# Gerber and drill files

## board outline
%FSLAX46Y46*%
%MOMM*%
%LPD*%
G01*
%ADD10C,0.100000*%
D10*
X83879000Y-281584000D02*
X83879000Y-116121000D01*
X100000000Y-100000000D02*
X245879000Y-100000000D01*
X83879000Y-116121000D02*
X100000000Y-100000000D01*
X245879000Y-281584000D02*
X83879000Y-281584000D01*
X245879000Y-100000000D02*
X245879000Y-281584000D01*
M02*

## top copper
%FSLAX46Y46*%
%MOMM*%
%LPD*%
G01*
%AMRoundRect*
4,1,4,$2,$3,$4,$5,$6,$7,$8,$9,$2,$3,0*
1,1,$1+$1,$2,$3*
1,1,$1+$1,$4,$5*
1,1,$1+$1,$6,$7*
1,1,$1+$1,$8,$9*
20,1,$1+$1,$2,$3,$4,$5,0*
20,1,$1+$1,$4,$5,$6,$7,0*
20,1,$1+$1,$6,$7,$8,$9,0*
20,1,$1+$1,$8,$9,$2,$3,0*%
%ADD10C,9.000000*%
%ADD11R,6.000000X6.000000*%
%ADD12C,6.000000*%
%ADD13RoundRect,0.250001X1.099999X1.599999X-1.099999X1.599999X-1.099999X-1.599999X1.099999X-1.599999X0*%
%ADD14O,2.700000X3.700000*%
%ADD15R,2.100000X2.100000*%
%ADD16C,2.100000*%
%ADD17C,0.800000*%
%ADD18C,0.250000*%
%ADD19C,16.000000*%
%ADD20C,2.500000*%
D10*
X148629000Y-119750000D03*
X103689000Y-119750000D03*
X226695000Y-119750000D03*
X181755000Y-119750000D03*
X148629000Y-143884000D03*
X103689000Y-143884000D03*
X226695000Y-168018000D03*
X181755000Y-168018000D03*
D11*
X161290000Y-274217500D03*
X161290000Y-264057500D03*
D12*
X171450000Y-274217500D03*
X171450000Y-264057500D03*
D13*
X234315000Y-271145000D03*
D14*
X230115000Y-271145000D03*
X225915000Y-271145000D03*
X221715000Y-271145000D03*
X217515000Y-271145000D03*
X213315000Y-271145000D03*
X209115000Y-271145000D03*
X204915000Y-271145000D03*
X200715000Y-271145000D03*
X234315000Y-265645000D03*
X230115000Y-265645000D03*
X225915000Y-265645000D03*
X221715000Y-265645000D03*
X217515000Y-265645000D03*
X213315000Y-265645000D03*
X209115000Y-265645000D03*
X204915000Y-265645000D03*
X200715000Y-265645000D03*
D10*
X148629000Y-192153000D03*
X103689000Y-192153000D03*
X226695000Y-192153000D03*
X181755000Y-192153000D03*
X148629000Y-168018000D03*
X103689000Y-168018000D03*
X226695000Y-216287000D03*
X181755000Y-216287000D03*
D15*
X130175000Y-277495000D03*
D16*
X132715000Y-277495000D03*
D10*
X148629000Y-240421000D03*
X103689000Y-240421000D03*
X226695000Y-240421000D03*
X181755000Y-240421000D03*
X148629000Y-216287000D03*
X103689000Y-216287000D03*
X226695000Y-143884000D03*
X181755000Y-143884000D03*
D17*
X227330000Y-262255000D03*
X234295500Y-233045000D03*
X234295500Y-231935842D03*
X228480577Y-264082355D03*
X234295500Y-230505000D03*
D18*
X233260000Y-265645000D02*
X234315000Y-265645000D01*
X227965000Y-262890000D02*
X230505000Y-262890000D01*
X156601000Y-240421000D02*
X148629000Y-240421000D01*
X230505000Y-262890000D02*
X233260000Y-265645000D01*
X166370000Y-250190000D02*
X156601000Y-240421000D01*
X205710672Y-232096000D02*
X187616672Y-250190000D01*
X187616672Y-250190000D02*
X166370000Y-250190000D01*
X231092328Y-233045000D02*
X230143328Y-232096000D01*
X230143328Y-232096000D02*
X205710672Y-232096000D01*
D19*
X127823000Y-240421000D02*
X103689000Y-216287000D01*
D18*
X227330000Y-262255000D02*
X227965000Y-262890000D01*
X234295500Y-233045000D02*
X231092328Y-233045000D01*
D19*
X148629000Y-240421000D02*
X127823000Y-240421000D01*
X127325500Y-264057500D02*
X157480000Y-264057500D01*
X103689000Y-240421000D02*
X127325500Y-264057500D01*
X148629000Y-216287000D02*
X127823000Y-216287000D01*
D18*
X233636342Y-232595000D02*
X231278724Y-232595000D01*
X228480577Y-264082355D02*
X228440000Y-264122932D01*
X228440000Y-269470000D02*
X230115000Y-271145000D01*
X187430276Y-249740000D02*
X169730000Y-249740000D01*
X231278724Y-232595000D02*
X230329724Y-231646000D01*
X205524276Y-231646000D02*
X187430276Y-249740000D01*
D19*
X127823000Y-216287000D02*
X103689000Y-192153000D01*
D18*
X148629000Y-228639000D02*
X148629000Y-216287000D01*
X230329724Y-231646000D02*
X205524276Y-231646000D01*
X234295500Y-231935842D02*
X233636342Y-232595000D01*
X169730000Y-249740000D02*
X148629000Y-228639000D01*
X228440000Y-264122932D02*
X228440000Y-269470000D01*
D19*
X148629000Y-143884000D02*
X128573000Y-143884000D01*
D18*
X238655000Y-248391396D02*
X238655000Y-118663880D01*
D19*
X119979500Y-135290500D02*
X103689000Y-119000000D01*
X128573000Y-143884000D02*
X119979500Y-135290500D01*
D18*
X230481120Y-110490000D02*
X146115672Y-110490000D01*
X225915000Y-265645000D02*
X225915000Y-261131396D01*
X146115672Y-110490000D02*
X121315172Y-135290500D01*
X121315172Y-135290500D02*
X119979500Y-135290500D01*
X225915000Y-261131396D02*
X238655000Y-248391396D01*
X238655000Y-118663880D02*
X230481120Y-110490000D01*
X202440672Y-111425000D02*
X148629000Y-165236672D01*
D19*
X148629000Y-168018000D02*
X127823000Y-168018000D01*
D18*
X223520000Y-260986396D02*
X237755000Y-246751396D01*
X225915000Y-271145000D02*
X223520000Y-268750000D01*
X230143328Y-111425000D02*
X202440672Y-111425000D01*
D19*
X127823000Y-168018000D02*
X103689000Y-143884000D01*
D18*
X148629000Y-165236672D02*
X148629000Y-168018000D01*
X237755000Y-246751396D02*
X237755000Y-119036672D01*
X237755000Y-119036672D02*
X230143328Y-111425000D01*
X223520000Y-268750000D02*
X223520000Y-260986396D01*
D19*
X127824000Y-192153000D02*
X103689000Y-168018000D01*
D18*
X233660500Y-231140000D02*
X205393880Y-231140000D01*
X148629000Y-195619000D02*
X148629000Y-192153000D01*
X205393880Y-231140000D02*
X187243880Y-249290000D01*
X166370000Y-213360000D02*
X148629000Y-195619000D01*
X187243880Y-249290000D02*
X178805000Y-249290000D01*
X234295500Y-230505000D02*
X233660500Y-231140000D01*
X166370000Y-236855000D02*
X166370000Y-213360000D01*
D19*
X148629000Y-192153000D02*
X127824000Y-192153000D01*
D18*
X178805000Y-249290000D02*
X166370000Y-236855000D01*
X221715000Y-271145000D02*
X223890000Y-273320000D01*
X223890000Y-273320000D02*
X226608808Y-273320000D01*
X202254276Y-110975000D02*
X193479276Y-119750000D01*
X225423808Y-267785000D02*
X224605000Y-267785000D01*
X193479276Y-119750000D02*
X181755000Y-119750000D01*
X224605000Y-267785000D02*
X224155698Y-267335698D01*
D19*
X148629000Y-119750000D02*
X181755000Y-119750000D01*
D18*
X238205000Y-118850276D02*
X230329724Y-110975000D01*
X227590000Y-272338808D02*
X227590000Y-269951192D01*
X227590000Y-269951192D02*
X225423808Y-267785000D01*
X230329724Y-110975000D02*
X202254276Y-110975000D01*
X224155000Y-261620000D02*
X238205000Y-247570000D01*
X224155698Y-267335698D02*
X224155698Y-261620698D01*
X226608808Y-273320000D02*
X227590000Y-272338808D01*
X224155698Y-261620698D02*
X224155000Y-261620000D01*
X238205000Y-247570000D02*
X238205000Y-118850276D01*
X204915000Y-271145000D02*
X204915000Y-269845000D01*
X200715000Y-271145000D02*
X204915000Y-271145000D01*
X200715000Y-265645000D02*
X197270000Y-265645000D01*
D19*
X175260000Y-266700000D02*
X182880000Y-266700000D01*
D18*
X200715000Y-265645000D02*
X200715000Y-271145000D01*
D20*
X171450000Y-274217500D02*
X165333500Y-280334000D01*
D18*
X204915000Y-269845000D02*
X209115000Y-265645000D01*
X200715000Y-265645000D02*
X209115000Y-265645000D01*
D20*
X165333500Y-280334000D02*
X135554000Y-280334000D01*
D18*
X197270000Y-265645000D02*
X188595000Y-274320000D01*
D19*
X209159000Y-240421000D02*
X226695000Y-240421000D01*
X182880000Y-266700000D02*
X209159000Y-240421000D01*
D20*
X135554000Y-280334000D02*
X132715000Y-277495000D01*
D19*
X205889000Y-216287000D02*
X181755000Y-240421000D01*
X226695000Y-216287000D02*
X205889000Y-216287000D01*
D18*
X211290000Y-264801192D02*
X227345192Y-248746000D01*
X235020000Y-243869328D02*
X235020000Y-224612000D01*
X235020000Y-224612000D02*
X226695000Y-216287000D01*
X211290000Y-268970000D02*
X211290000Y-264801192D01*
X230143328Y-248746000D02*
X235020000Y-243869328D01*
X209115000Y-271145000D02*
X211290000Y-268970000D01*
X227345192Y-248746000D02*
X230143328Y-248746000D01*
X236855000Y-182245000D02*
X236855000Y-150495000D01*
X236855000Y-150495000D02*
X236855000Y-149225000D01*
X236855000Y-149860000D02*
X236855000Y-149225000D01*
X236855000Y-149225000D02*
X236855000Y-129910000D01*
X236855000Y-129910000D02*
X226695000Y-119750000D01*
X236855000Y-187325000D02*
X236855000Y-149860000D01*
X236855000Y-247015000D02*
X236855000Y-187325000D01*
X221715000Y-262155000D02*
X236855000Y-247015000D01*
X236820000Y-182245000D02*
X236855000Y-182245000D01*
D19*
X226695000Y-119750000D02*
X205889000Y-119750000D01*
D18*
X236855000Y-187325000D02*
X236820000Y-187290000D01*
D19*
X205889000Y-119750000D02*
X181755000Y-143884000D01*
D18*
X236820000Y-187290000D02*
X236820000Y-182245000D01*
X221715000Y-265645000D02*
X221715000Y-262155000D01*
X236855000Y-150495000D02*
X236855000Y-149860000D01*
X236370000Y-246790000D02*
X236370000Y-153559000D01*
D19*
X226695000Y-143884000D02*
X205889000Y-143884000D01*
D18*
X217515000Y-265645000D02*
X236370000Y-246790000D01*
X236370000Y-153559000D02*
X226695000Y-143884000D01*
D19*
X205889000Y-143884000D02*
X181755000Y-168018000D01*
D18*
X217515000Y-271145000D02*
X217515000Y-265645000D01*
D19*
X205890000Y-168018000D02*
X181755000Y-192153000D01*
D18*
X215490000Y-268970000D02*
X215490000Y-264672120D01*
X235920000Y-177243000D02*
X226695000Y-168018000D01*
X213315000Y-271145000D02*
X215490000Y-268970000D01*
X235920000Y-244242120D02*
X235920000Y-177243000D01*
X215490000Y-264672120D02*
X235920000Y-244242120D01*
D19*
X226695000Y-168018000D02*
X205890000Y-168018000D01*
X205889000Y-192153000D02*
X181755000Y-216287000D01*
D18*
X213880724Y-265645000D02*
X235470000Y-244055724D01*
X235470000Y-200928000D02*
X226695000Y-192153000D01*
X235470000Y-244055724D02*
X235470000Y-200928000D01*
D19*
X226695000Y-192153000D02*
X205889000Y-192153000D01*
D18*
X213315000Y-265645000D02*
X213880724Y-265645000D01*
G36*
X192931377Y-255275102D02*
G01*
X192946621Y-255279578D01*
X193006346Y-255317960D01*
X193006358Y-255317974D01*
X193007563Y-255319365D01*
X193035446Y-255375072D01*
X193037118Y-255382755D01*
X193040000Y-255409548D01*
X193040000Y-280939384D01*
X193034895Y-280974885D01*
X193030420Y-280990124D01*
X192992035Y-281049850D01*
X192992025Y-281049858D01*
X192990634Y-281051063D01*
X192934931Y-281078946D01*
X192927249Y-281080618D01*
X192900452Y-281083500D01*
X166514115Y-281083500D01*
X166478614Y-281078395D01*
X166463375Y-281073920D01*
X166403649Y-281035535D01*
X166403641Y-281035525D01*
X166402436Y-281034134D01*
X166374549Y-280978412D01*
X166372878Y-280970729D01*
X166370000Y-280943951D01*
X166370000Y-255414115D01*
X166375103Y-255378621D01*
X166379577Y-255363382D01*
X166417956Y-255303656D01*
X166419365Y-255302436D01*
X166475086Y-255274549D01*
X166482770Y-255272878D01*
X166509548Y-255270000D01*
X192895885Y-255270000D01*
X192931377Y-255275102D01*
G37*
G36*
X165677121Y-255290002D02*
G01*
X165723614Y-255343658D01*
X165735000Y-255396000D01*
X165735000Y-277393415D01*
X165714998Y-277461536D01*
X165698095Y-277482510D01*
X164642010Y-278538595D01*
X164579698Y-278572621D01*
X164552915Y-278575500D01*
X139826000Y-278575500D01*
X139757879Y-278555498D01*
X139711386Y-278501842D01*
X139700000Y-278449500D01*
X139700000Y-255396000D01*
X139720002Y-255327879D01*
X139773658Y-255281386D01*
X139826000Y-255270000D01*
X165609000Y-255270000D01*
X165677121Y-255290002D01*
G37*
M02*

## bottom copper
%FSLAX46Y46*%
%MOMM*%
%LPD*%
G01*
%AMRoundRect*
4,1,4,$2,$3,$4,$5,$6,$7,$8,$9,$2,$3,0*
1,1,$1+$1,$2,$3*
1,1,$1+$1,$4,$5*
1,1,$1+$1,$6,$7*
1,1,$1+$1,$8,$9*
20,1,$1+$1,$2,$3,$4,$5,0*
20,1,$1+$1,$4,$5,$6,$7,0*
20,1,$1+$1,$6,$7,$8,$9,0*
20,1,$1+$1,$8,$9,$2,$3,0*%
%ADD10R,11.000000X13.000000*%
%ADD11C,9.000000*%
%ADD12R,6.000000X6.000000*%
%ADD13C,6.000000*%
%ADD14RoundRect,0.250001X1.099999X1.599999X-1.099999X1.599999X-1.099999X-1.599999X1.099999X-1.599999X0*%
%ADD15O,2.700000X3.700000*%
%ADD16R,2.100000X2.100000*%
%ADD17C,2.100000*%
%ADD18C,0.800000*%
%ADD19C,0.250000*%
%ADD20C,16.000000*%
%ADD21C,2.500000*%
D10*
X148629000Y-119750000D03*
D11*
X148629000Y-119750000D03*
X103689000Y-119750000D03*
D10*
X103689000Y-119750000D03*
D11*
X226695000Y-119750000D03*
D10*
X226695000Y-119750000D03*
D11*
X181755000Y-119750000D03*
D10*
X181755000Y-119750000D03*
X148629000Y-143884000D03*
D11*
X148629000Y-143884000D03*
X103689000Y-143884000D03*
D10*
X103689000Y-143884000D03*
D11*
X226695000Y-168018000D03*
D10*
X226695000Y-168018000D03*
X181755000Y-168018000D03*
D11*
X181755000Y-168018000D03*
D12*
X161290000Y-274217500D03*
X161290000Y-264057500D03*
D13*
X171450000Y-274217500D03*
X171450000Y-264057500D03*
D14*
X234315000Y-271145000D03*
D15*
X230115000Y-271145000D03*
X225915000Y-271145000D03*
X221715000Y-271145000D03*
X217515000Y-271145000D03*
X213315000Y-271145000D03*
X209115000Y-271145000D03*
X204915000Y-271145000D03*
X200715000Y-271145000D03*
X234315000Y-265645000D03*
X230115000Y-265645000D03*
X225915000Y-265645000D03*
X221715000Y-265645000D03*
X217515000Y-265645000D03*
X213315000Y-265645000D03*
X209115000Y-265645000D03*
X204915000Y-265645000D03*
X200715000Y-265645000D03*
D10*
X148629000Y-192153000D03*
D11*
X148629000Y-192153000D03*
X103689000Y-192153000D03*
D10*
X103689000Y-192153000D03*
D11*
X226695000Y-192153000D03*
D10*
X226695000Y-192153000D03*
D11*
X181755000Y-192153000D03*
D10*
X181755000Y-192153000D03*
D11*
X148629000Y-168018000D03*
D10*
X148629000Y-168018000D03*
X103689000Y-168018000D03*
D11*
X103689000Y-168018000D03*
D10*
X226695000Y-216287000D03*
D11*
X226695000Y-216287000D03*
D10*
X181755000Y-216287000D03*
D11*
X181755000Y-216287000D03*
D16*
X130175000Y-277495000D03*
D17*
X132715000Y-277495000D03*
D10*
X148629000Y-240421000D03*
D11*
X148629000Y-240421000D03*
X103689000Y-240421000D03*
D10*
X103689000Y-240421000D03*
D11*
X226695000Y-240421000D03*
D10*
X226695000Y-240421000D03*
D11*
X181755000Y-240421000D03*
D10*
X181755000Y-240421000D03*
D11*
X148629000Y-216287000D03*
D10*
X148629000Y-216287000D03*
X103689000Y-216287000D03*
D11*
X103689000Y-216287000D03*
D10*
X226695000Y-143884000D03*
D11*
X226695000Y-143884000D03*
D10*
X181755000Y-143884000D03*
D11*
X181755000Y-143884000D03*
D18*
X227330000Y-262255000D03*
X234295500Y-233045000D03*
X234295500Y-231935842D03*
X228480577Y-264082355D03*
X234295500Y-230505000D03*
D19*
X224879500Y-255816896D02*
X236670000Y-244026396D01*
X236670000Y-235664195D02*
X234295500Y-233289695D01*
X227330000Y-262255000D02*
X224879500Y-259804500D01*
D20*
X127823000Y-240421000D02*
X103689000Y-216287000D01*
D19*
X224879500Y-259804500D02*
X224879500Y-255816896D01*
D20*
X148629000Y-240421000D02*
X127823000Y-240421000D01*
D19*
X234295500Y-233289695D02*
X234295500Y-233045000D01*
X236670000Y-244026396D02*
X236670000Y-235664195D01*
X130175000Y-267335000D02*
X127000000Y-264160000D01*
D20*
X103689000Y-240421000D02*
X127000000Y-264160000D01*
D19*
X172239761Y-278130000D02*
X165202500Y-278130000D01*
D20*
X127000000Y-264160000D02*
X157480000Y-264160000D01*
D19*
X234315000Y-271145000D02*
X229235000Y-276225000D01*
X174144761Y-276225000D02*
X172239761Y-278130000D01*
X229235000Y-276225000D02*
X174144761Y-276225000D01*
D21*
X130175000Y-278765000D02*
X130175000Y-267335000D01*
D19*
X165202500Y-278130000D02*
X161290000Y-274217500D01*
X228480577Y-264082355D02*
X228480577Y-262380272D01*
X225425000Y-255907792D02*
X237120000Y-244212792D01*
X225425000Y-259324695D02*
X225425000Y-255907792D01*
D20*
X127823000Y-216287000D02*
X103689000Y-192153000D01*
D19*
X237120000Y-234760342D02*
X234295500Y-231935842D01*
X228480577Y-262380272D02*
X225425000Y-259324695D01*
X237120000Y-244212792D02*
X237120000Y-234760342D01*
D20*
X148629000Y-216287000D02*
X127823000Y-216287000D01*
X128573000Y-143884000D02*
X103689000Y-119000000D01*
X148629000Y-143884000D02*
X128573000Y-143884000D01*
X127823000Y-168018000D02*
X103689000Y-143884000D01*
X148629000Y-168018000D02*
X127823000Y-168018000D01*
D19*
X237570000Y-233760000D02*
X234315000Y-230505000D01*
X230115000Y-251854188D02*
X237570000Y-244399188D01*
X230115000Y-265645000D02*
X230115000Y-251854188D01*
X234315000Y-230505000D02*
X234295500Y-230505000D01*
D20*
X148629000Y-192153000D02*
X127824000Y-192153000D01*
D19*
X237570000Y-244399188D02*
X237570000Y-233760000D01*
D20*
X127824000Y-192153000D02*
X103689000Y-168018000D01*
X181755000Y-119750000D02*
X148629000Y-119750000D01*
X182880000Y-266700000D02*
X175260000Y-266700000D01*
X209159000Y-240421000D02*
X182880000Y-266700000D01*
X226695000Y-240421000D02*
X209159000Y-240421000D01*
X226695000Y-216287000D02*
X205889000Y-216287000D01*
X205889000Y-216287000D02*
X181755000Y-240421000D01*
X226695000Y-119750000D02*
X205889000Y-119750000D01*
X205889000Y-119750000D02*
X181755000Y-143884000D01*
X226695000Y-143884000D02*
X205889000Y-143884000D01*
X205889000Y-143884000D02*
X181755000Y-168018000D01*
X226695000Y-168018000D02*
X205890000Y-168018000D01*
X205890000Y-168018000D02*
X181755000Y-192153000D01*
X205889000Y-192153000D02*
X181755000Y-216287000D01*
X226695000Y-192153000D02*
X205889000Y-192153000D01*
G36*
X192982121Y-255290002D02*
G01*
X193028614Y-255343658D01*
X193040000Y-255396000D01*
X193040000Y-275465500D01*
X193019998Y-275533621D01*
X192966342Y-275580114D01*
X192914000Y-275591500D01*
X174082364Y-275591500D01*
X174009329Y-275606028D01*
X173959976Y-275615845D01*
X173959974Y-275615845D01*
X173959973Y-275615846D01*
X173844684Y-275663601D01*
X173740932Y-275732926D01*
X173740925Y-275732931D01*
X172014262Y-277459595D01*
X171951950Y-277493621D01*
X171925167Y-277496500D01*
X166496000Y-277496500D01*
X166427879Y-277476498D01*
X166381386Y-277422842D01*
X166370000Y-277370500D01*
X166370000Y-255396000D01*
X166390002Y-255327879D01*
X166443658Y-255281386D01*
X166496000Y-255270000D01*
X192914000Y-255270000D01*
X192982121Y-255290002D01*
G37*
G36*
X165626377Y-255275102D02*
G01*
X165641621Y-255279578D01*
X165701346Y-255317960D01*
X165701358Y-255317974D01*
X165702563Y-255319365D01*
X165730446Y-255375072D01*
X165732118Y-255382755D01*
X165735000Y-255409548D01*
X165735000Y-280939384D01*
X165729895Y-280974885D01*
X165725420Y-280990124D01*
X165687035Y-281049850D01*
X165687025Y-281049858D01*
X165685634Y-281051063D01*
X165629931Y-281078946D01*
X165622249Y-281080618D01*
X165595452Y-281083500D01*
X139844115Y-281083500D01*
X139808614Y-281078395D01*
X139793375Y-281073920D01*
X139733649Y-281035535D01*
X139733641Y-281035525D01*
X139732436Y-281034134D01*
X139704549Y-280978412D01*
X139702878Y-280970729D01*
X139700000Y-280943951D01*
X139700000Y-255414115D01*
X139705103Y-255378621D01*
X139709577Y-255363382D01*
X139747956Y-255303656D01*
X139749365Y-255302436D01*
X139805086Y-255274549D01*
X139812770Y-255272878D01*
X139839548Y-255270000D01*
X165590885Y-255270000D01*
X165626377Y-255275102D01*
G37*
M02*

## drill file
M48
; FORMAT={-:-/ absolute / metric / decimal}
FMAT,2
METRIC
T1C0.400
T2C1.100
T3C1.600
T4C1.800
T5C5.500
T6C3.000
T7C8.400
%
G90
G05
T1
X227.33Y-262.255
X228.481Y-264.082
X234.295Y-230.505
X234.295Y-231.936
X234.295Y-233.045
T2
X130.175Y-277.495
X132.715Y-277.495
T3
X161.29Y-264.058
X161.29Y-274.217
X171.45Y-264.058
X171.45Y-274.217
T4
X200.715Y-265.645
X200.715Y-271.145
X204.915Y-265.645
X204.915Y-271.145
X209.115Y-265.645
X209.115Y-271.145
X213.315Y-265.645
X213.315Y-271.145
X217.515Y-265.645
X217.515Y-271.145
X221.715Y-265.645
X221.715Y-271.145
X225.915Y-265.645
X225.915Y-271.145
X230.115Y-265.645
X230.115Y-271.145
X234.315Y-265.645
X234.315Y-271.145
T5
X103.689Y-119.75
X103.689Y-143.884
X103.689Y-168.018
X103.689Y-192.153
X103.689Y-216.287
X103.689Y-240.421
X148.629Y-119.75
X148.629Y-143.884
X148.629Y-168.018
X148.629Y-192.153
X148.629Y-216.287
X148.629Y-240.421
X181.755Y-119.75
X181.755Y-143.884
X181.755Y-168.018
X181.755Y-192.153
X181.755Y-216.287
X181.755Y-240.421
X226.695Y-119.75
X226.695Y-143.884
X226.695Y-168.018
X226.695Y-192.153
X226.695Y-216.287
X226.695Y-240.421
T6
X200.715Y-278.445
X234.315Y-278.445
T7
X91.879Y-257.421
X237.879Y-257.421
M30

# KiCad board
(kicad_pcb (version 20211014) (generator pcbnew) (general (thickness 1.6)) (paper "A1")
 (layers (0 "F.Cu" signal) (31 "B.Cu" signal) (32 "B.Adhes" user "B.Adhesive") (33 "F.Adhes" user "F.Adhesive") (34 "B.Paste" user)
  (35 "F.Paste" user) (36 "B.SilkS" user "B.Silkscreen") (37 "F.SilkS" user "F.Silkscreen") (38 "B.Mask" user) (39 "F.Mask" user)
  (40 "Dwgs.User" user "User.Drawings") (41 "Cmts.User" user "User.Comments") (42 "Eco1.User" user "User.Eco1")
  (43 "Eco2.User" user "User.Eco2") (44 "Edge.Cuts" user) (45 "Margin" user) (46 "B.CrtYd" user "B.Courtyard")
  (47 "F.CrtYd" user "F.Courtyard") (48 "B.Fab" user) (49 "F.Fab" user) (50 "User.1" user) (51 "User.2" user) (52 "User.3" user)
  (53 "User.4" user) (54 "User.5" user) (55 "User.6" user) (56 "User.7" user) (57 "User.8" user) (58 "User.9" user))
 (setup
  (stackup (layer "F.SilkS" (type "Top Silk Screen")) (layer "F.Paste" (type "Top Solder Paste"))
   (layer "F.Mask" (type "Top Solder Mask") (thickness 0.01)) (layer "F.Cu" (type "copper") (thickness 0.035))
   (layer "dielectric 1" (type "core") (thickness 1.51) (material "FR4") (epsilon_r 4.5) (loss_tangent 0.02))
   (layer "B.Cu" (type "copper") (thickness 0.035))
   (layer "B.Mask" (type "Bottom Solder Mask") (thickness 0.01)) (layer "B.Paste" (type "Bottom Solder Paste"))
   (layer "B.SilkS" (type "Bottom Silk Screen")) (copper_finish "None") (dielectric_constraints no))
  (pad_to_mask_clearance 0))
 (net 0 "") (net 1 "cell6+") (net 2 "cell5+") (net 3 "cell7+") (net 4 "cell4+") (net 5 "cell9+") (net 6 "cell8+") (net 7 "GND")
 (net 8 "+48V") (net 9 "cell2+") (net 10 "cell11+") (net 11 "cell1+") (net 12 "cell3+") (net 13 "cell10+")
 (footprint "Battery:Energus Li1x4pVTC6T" (layer "F.Cu") (at 148.629 119.75 180)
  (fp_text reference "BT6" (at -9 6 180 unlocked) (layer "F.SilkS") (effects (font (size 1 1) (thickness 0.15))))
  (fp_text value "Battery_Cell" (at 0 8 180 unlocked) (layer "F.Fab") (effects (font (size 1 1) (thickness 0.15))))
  (pad "1" smd rect (at 0 0 180) (size 11 13) (layers "B.Cu" "B.Paste" "B.Mask") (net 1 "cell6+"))
  (pad "1" thru_hole circle (at 0 0 180) (size 9 9) (drill 5.5) (layers *.Cu *.Mask) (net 1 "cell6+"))
  (pad "2" thru_hole circle (at 44.94 0 180) (size 9 9) (drill 5.5) (layers *.Cu *.Mask) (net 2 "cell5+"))
  (pad "2" smd rect (at 44.94 0 180) (size 11 13) (layers "B.Cu" "B.Paste" "B.Mask") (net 2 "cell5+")))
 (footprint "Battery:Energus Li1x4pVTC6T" (layer "F.Cu") (at 226.695 119.75 180)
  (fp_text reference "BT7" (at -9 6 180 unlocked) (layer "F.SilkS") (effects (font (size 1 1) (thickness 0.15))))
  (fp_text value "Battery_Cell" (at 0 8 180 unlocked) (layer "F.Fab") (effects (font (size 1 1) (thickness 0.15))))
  (pad "1" thru_hole circle (at 0 0 180) (size 9 9) (drill 5.5) (layers *.Cu *.Mask) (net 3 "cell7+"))
  (pad "1" smd rect (at 0 0 180) (size 11 13) (layers "B.Cu" "B.Paste" "B.Mask") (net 3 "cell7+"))
  (pad "2" thru_hole circle (at 44.94 0 180) (size 9 9) (drill 5.5) (layers *.Cu *.Mask) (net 1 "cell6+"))
  (pad "2" smd rect (at 44.94 0 180) (size 11 13) (layers "B.Cu" "B.Paste" "B.Mask") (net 1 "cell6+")))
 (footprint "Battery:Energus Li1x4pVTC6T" (layer "F.Cu") (at 148.629 143.884 180)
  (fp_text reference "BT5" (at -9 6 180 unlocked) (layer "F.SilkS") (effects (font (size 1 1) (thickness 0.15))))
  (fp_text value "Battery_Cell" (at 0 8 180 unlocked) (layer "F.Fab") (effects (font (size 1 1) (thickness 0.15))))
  (pad "1" smd rect (at 0 0 180) (size 11 13) (layers "B.Cu" "B.Paste" "B.Mask") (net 2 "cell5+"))
  (pad "1" thru_hole circle (at 0 0 180) (size 9 9) (drill 5.5) (layers *.Cu *.Mask) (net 2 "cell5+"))
  (pad "2" thru_hole circle (at 44.94 0 180) (size 9 9) (drill 5.5) (layers *.Cu *.Mask) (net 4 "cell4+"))
  (pad "2" smd rect (at 44.94 0 180) (size 11 13) (layers "B.Cu" "B.Paste" "B.Mask") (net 4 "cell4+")))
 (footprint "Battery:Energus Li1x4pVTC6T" (layer "F.Cu") (at 226.695 168.018 180)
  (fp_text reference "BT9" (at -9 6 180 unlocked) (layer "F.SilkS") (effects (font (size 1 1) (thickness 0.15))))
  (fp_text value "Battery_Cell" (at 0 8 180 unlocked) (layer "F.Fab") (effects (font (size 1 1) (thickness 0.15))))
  (pad "1" thru_hole circle (at 0 0 180) (size 9 9) (drill 5.5) (layers *.Cu *.Mask) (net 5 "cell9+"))
  (pad "1" smd rect (at 0 0 180) (size 11 13) (layers "B.Cu" "B.Paste" "B.Mask") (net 5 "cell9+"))
  (pad "2" smd rect (at 44.94 0 180) (size 11 13) (layers "B.Cu" "B.Paste" "B.Mask") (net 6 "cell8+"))
  (pad "2" thru_hole circle (at 44.94 0 180) (size 9 9) (drill 5.5) (layers *.Cu *.Mask) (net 6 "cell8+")))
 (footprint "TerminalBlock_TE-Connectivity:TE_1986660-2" (layer "F.Cu") (at 161.29 264.0575)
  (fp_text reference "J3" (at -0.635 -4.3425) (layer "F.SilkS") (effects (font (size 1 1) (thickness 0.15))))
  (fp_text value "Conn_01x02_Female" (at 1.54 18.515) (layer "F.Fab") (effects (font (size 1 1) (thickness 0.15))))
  (pad "1" thru_hole rect (at 0 10.16) (size 6 6) (drill 1.6) (layers *.Cu *.Mask) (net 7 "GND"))
  (pad "1" thru_hole rect (at 0 0) (size 6 6) (drill 1.6) (layers *.Cu *.Mask) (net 7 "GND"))
  (pad "2" thru_hole circle (at 10.16 10.16) (size 6 6) (drill 1.6) (layers *.Cu *.Mask) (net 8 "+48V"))
  (pad "2" thru_hole circle (at 10.16 0) (size 6 6) (drill 1.6) (layers *.Cu *.Mask) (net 8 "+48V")))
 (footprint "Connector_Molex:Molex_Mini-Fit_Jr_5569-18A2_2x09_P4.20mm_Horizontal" (layer "F.Cu") (at 234.315 271.145 180)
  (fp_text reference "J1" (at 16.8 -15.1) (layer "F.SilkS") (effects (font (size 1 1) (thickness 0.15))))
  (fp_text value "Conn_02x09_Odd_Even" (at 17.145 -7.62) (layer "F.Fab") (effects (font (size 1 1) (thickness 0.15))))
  (pad "" np_thru_hole circle (at 0 -7.3 180) (size 3 3) (drill 3) (layers *.Cu *.Mask))
  (pad "" np_thru_hole circle (at 33.6 -7.3 180) (size 3 3) (drill 3) (layers *.Cu *.Mask))
  (pad "1" thru_hole roundrect (at 0 0 180) (size 2.7 3.7) (drill 1.8) (layers *.Cu *.Mask) (roundrect_rratio 0.092593) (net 7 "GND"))
  (pad "2" thru_hole oval (at 4.2 0 180) (size 2.7 3.7) (drill 1.8) (layers *.Cu *.Mask) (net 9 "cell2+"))
  (pad "3" thru_hole oval (at 8.4 0 180) (size 2.7 3.7) (drill 1.8) (layers *.Cu *.Mask) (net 4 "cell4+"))
  (pad "4" thru_hole oval (at 12.6 0 180) (size 2.7 3.7) (drill 1.8) (layers *.Cu *.Mask) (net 1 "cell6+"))
  (pad "5" thru_hole oval (at 16.8 0 180) (size 2.7 3.7) (drill 1.8) (layers *.Cu *.Mask) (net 6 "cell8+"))
  (pad "6" thru_hole oval (at 21 0 180) (size 2.7 3.7) (drill 1.8) (layers *.Cu *.Mask) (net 5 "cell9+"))
  (pad "7" thru_hole oval (at 25.2 0 180) (size 2.7 3.7) (drill 1.8) (layers *.Cu *.Mask) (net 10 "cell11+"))
  (pad "8" thru_hole oval (at 29.4 0 180) (size 2.7 3.7) (drill 1.8) (layers *.Cu *.Mask) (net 8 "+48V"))
  (pad "9" thru_hole oval (at 33.6 0 180) (size 2.7 3.7) (drill 1.8) (layers *.Cu *.Mask) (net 8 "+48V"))
  (pad "10" thru_hole oval (at 0 5.5 180) (size 2.7 3.7) (drill 1.8) (layers *.Cu *.Mask) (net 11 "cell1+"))
  (pad "11" thru_hole oval (at 4.2 5.5 180) (size 2.7 3.7) (drill 1.8) (layers *.Cu *.Mask) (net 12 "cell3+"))
  (pad "12" thru_hole oval (at 8.4 5.5 180) (size 2.7 3.7) (drill 1.8) (layers *.Cu *.Mask) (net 2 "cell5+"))
  (pad "13" thru_hole oval (at 12.6 5.5 180) (size 2.7 3.7) (drill 1.8) (layers *.Cu *.Mask) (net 3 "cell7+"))
  (pad "14" thru_hole oval (at 16.8 5.5 180) (size 2.7 3.7) (drill 1.8) (layers *.Cu *.Mask) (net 6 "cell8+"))
  (pad "15" thru_hole oval (at 21 5.5 180) (size 2.7 3.7) (drill 1.8) (layers *.Cu *.Mask) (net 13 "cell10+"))
  (pad "16" thru_hole oval (at 25.2 5.5 180) (size 2.7 3.7) (drill 1.8) (layers *.Cu *.Mask) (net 8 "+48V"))
  (pad "17" thru_hole oval (at 29.4 5.5 180) (size 2.7 3.7) (drill 1.8) (layers *.Cu *.Mask) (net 8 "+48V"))
  (pad "18" thru_hole oval (at 33.6 5.5 180) (size 2.7 3.7) (drill 1.8) (layers *.Cu *.Mask) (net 8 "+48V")))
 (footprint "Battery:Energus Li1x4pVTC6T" (layer "F.Cu") (at 148.629 192.153 180)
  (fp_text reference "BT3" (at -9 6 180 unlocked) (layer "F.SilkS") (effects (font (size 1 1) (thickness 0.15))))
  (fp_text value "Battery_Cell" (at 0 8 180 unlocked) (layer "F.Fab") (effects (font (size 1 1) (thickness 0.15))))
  (pad "1" smd rect (at 0 0 180) (size 11 13) (layers "B.Cu" "B.Paste" "B.Mask") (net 12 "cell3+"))
  (pad "1" thru_hole circle (at 0 0 180) (size 9 9) (drill 5.5) (layers *.Cu *.Mask) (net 12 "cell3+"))
  (pad "2" thru_hole circle (at 44.94 0 180) (size 9 9) (drill 5.5) (layers *.Cu *.Mask) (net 9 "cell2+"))
  (pad "2" smd rect (at 44.94 0 180) (size 11 13) (layers "B.Cu" "B.Paste" "B.Mask") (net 9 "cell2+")))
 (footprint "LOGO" (layer "F.Cu") (at 105.41 267.97)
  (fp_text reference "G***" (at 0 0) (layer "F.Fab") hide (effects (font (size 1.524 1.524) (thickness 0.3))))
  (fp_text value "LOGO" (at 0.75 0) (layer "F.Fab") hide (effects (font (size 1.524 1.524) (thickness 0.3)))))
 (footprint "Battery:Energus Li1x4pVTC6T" (layer "F.Cu") (at 226.695 192.153 180)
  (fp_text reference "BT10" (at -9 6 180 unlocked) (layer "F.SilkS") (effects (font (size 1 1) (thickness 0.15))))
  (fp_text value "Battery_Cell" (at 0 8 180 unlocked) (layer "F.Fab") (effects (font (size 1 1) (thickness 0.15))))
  (pad "1" thru_hole circle (at 0 0 180) (size 9 9) (drill 5.5) (layers *.Cu *.Mask) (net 13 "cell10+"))
  (pad "1" smd rect (at 0 0 180) (size 11 13) (layers "B.Cu" "B.Paste" "B.Mask") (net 13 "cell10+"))
  (pad "2" thru_hole circle (at 44.94 0 180) (size 9 9) (drill 5.5) (layers *.Cu *.Mask) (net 5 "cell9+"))
  (pad "2" smd rect (at 44.94 0 180) (size 11 13) (layers "B.Cu" "B.Paste" "B.Mask") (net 5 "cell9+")))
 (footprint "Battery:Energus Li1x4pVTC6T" (layer "F.Cu") (at 148.629 168.018 180)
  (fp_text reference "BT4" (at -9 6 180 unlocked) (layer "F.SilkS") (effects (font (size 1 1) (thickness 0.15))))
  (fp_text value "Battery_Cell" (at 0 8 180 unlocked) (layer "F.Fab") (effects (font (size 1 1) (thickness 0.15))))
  (pad "1" thru_hole circle (at 0 0 180) (size 9 9) (drill 5.5) (layers *.Cu *.Mask) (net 4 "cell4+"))
  (pad "1" smd rect (at 0 0 180) (size 11 13) (layers "B.Cu" "B.Paste" "B.Mask") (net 4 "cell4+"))
  (pad "2" smd rect (at 44.94 0 180) (size 11 13) (layers "B.Cu" "B.Paste" "B.Mask") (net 12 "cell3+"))
  (pad "2" thru_hole circle (at 44.94 0 180) (size 9 9) (drill 5.5) (layers *.Cu *.Mask) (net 12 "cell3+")))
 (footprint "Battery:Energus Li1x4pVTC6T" (layer "F.Cu") (at 226.695 216.287 180)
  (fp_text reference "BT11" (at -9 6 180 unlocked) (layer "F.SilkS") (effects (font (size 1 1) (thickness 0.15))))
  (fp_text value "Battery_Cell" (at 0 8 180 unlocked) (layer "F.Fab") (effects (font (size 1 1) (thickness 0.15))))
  (pad "1" smd rect (at 0 0 180) (size 11 13) (layers "B.Cu" "B.Paste" "B.Mask") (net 10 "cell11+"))
  (pad "1" thru_hole circle (at 0 0 180) (size 9 9) (drill 5.5) (layers *.Cu *.Mask) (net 10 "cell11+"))
  (pad "2" smd rect (at 44.94 0 180) (size 11 13) (layers "B.Cu" "B.Paste" "B.Mask") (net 13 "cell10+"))
  (pad "2" thru_hole circle (at 44.94 0 180) (size 9 9) (drill 5.5) (layers *.Cu *.Mask) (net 13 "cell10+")))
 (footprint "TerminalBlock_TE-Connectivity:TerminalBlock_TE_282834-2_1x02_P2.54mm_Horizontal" (layer "F.Cu") (at 130.175 277.495)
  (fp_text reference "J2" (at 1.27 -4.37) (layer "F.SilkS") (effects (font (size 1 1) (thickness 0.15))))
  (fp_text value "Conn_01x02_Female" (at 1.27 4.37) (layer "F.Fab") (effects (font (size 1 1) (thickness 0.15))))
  (pad "1" thru_hole rect (at 0 0) (size 2.1 2.1) (drill 1.1) (layers *.Cu *.Mask) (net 7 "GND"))
  (pad "2" thru_hole circle (at 2.54 0) (size 2.1 2.1) (drill 1.1) (layers *.Cu *.Mask) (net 8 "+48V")))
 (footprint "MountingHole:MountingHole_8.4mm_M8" (layer "F.Cu") (at 237.879 257.421)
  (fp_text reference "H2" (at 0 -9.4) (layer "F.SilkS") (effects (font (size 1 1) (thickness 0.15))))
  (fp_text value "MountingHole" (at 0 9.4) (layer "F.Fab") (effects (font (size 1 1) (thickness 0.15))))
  (pad "" np_thru_hole circle (at 0 0) (size 8.4 8.4) (drill 8.4) (layers *.Cu *.Mask)))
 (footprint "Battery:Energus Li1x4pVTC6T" (layer "F.Cu") (at 148.629 240.421 180)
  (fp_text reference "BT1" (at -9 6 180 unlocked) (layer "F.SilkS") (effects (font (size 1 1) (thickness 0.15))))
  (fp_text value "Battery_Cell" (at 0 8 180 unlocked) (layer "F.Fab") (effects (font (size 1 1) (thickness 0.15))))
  (pad "1" smd rect (at 0 0 180) (size 11 13) (layers "B.Cu" "B.Paste" "B.Mask") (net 11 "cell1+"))
  (pad "1" thru_hole circle (at 0 0 180) (size 9 9) (drill 5.5) (layers *.Cu *.Mask) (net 11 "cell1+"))
  (pad "2" thru_hole circle (at 44.94 0 180) (size 9 9) (drill 5.5) (layers *.Cu *.Mask) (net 7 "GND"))
  (pad "2" smd rect (at 44.94 0 180) (size 11 13) (layers "B.Cu" "B.Paste" "B.Mask") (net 7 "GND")))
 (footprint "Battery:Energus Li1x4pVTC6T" (layer "F.Cu") (at 226.695 240.421 180)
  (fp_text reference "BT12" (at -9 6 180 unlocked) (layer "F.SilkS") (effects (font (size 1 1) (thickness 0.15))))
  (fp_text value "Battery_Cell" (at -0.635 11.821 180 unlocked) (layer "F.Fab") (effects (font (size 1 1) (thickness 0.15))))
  (pad "1" thru_hole circle (at 0 0 180) (size 9 9) (drill 5.5) (layers *.Cu *.Mask) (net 8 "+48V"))
  (pad "1" smd rect (at 0 0 180) (size 11 13) (layers "B.Cu" "B.Paste" "B.Mask") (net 8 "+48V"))
  (pad "2" thru_hole circle (at 44.94 0 180) (size 9 9) (drill 5.5) (layers *.Cu *.Mask) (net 10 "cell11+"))
  (pad "2" smd rect (at 44.94 0 180) (size 11 13) (layers "B.Cu" "B.Paste" "B.Mask") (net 10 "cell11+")))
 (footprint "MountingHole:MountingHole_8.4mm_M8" (layer "F.Cu") (at 91.879 257.421)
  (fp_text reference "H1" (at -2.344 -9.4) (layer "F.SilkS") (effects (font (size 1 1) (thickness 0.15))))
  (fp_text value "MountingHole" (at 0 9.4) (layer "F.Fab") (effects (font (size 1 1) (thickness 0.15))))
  (pad "" np_thru_hole circle (at 0 0) (size 8.4 8.4) (drill 8.4) (layers *.Cu *.Mask)))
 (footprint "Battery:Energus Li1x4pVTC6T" (layer "F.Cu") (at 148.629 216.287 180)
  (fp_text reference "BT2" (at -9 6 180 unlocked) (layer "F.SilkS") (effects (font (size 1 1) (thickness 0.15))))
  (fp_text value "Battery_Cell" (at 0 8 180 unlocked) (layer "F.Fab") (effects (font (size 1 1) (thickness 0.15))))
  (pad "1" thru_hole circle (at 0 0 180) (size 9 9) (drill 5.5) (layers *.Cu *.Mask) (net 9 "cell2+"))
  (pad "1" smd rect (at 0 0 180) (size 11 13) (layers "B.Cu" "B.Paste" "B.Mask") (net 9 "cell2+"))
  (pad "2" smd rect (at 44.94 0 180) (size 11 13) (layers "B.Cu" "B.Paste" "B.Mask") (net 11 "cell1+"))
  (pad "2" thru_hole circle (at 44.94 0 180) (size 9 9) (drill 5.5) (layers *.Cu *.Mask) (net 11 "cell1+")))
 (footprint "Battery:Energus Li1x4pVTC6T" (layer "F.Cu") (at 226.695 143.884 180)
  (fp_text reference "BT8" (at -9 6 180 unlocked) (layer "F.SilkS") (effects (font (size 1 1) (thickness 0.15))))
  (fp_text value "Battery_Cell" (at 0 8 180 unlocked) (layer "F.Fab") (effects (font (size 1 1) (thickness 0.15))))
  (pad "1" smd rect (at 0 0 180) (size 11 13) (layers "B.Cu" "B.Paste" "B.Mask") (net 6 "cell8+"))
  (pad "1" thru_hole circle (at 0 0 180) (size 9 9) (drill 5.5) (layers *.Cu *.Mask) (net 6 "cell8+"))
  (pad "2" smd rect (at 44.94 0 180) (size 11 13) (layers "B.Cu" "B.Paste" "B.Mask") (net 3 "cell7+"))
  (pad "2" thru_hole circle (at 44.94 0 180) (size 9 9) (drill 5.5) (layers *.Cu *.Mask) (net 3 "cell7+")))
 (gr_line (start 83.879 281.584) (end 83.879 116.121) (layer "Edge.Cuts") (width 0.1))
 (gr_line (start 100 100) (end 245.879 100) (layer "Edge.Cuts") (width 0.1))
 (gr_line (start 83.879 116.121) (end 100 100) (layer "Edge.Cuts") (width 0.1))
 (gr_line (start 245.879 281.584) (end 83.879 281.584) (layer "Edge.Cuts") (width 0.1))
 (gr_line (start 245.879 100) (end 245.879 281.584) (layer "Edge.Cuts") (width 0.1))
 (segment (start 233.26 265.645) (end 234.315 265.645) (width 0.25) (layer "F.Cu") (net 11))
 (segment (start 227.965 262.89) (end 230.505 262.89) (width 0.25) (layer "F.Cu") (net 11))
 (segment (start 156.601 240.421) (end 148.629 240.421) (width 0.25) (layer "F.Cu") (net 11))
 (segment (start 230.505 262.89) (end 233.26 265.645) (width 0.25) (layer "F.Cu") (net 11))
 (segment (start 166.37 250.19) (end 156.601 240.421) (width 0.25) (layer "F.Cu") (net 11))
 (segment (start 205.710672 232.096) (end 187.616672 250.19) (width 0.25) (layer "F.Cu") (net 11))
 (segment (start 187.616672 250.19) (end 166.37 250.19) (width 0.25) (layer "F.Cu") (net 11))
 (segment (start 231.092328 233.045) (end 230.143328 232.096) (width 0.25) (layer "F.Cu") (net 11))
 (segment (start 230.143328 232.096) (end 205.710672 232.096) (width 0.25) (layer "F.Cu") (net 11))
 (segment (start 127.823 240.421) (end 103.689 216.287) (width 16) (layer "F.Cu") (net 11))
 (segment (start 227.33 262.255) (end 227.965 262.89) (width 0.25) (layer "F.Cu") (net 11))
 (segment (start 234.2955 233.045) (end 231.092328 233.045) (width 0.25) (layer "F.Cu") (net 11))
 (segment (start 148.629 240.421) (end 127.823 240.421) (width 16) (layer "F.Cu") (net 11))
 (via (at 227.33 262.255) (size 0.8) (drill 0.4) (layers "F.Cu" "B.Cu") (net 11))
 (via (at 234.2955 233.045) (size 0.8) (drill 0.4) (layers "F.Cu" "B.Cu") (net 11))
 (segment (start 224.8795 255.816896) (end 236.67 244.026396) (width 0.25) (layer "B.Cu") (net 11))
 (segment (start 236.67 235.664195) (end 234.2955 233.289695) (width 0.25) (layer "B.Cu") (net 11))
 (segment (start 227.33 262.255) (end 224.8795 259.8045) (width 0.25) (layer "B.Cu") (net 11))
 (segment (start 127.823 240.421) (end 103.689 216.287) (width 16) (layer "B.Cu") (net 11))
 (segment (start 224.8795 259.8045) (end 224.8795 255.816896) (width 0.25) (layer "B.Cu") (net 11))
 (segment (start 148.629 240.421) (end 127.823 240.421) (width 16) (layer "B.Cu") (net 11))
 (segment (start 234.2955 233.289695) (end 234.2955 233.045) (width 0.25) (layer "B.Cu") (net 11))
 (segment (start 236.67 244.026396) (end 236.67 235.664195) (width 0.25) (layer "B.Cu") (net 11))
 (segment (start 127.3255 264.0575) (end 157.48 264.0575) (width 16) (layer "F.Cu") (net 7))
 (segment (start 103.689 240.421) (end 127.3255 264.0575) (width 16) (layer "F.Cu") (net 7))
 (segment (start 130.175 267.335) (end 127 264.16) (width 0.25) (layer "B.Cu") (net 7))
 (segment (start 103.689 240.421) (end 127 264.16) (width 16) (layer "B.Cu") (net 7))
 (segment (start 172.239761 278.13) (end 165.2025 278.13) (width 0.25) (layer "B.Cu") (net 7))
 (segment (start 127 264.16) (end 157.48 264.16) (width 16) (layer "B.Cu") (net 7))
 (segment (start 234.315 271.145) (end 229.235 276.225) (width 0.25) (layer "B.Cu") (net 7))
 (segment (start 174.144761 276.225) (end 172.239761 278.13) (width 0.25) (layer "B.Cu") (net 7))
 (segment (start 229.235 276.225) (end 174.144761 276.225) (width 0.25) (layer "B.Cu") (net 7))
 (segment (start 130.175 278.765) (end 130.175 267.335) (width 2.5) (layer "B.Cu") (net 7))
 (segment (start 165.2025 278.13) (end 161.29 274.2175) (width 0.25) (layer "B.Cu") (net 7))
 (segment (start 148.629 216.287) (end 127.823 216.287) (width 16) (layer "F.Cu") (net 9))
 (segment (start 233.636342 232.595) (end 231.278724 232.595) (width 0.25) (layer "F.Cu") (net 9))
 (segment (start 228.480577 264.082355) (end 228.44 264.122932) (width 0.25) (layer "F.Cu") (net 9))
 (segment (start 228.44 269.47) (end 230.115 271.145) (width 0.25) (layer "F.Cu") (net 9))
 (segment (start 187.430276 249.74) (end 169.73 249.74) (width 0.25) (layer "F.Cu") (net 9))
 (segment (start 231.278724 232.595) (end 230.329724 231.646) (width 0.25) (layer "F.Cu") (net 9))
 (segment (start 205.524276 231.646) (end 187.430276 249.74) (width 0.25) (layer "F.Cu") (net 9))
 (segment (start 127.823 216.287) (end 103.689 192.153) (width 16) (layer "F.Cu") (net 9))
 (segment (start 148.629 228.639) (end 148.629 216.287) (width 0.25) (layer "F.Cu") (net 9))
 (segment (start 230.329724 231.646) (end 205.524276 231.646) (width 0.25) (layer "F.Cu") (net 9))
 (segment (start 234.2955 231.935842) (end 233.636342 232.595) (width 0.25) (layer "F.Cu") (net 9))
 (segment (start 169.73 249.74) (end 148.629 228.639) (width 0.25) (layer "F.Cu") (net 9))
 (segment (start 228.44 264.122932) (end 228.44 269.47) (width 0.25) (layer "F.Cu") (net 9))
 (via (at 234.2955 231.935842) (size 0.8) (drill 0.4) (layers "F.Cu" "B.Cu") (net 9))
 (via (at 228.480577 264.082355) (size 0.8) (drill 0.4) (layers "F.Cu" "B.Cu") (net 9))
 (segment (start 228.480577 264.082355) (end 228.480577 262.380272) (width 0.25) (layer "B.Cu") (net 9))
 (segment (start 225.425 255.907792) (end 237.12 244.212792) (width 0.25) (layer "B.Cu") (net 9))
 (segment (start 225.425 259.324695) (end 225.425 255.907792) (width 0.25) (layer "B.Cu") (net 9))
 (segment (start 127.823 216.287) (end 103.689 192.153) (width 16) (layer "B.Cu") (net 9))
 (segment (start 237.12 234.760342) (end 234.2955 231.935842) (width 0.25) (layer "B.Cu") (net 9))
 (segment (start 228.480577 262.380272) (end 225.425 259.324695) (width 0.25) (layer "B.Cu") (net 9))
 (segment (start 237.12 244.212792) (end 237.12 234.760342) (width 0.25) (layer "B.Cu") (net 9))
 (segment (start 148.629 216.287) (end 127.823 216.287) (width 16) (layer "B.Cu") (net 9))
 (segment (start 148.629 143.884) (end 128.573 143.884) (width 16) (layer "F.Cu") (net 2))
 (segment (start 238.655 248.391396) (end 238.655 118.66388) (width 0.25) (layer "F.Cu") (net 2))
 (segment (start 119.9795 135.2905) (end 103.689 119) (width 16) (layer "F.Cu") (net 2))
 (segment (start 128.573 143.884) (end 119.9795 135.2905) (width 16) (layer "F.Cu") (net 2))
 (segment (start 230.48112 110.49) (end 146.115672 110.49) (width 0.25) (layer "F.Cu") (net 2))
 (segment (start 225.915 265.645) (end 225.915 261.131396) (width 0.25) (layer "F.Cu") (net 2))
 (segment (start 146.115672 110.49) (end 121.315172 135.2905) (width 0.25) (layer "F.Cu") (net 2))
 (segment (start 121.315172 135.2905) (end 119.9795 135.2905) (width 0.25) (layer "F.Cu") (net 2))
 (segment (start 225.915 261.131396) (end 238.655 248.391396) (width 0.25) (layer "F.Cu") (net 2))
 (segment (start 238.655 118.66388) (end 230.48112 110.49) (width 0.25) (layer "F.Cu") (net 2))
 (segment (start 128.573 143.884) (end 103.689 119) (width 16) (layer "B.Cu") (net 2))
 (segment (start 148.629 143.884) (end 128.573 143.884) (width 16) (layer "B.Cu") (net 2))
 (segment (start 202.440672 111.425) (end 148.629 165.236672) (width 0.25) (layer "F.Cu") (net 4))
 (segment (start 148.629 168.018) (end 127.823 168.018) (width 16) (layer "F.Cu") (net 4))
 (segment (start 223.52 260.986396) (end 237.755 246.751396) (width 0.25) (layer "F.Cu") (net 4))
 (segment (start 225.915 271.145) (end 223.52 268.75) (width 0.25) (layer "F.Cu") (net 4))
 (segment (start 230.143328 111.425) (end 202.440672 111.425) (width 0.25) (layer "F.Cu") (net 4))
 (segment (start 127.823 168.018) (end 103.689 143.884) (width 16) (layer "F.Cu") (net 4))
 (segment (start 148.629 165.236672) (end 148.629 168.018) (width 0.25) (layer "F.Cu") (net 4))
 (segment (start 237.755 246.751396) (end 237.755 119.036672) (width 0.25) (layer "F.Cu") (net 4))
 (segment (start 237.755 119.036672) (end 230.143328 111.425) (width 0.25) (layer "F.Cu") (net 4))
 (segment (start 223.52 268.75) (end 223.52 260.986396) (width 0.25) (layer "F.Cu") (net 4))
 (segment (start 127.823 168.018) (end 103.689 143.884) (width 16) (layer "B.Cu") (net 4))
 (segment (start 148.629 168.018) (end 127.823 168.018) (width 16) (layer "B.Cu") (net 4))
 (segment (start 127.824 192.153) (end 103.689 168.018) (width 16) (layer "F.Cu") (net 12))
 (segment (start 233.6605 231.14) (end 205.39388 231.14) (width 0.25) (layer "F.Cu") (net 12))
 (segment (start 148.629 195.619) (end 148.629 192.153) (width 0.25) (layer "F.Cu") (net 12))
 (segment (start 205.39388 231.14) (end 187.24388 249.29) (width 0.25) (layer "F.Cu") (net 12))
 (segment (start 166.37 213.36) (end 148.629 195.619) (width 0.25) (layer "F.Cu") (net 12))
 (segment (start 187.24388 249.29) (end 178.805 249.29) (width 0.25) (layer "F.Cu") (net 12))
 (segment (start 234.2955 230.505) (end 233.6605 231.14) (width 0.25) (layer "F.Cu") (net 12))
 (segment (start 166.37 236.855) (end 166.37 213.36) (width 0.25) (layer "F.Cu") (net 12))
 (segment (start 148.629 192.153) (end 127.824 192.153) (width 16) (layer "F.Cu") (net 12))
 (segment (start 178.805 249.29) (end 166.37 236.855) (width 0.25) (layer "F.Cu") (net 12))
 (via (at 234.2955 230.505) (size 0.8) (drill 0.4) (layers "F.Cu" "B.Cu") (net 12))
 (segment (start 237.57 233.76) (end 234.315 230.505) (width 0.25) (layer "B.Cu") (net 12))
 (segment (start 230.115 251.854188) (end 237.57 244.399188) (width 0.25) (layer "B.Cu") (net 12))
 (segment (start 230.115 265.645) (end 230.115 251.854188) (width 0.25) (layer "B.Cu") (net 12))
 (segment (start 234.315 230.505) (end 234.2955 230.505) (width 0.25) (layer "B.Cu") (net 12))
 (segment (start 148.629 192.153) (end 127.824 192.153) (width 16) (layer "B.Cu") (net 12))
 (segment (start 237.57 244.399188) (end 237.57 233.76) (width 0.25) (layer "B.Cu") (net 12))
 (segment (start 127.824 192.153) (end 103.689 168.018) (width 16) (layer "B.Cu") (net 12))
 (segment (start 221.715 271.145) (end 223.89 273.32) (width 0.25) (layer "F.Cu") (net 1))
 (segment (start 223.89 273.32) (end 226.608808 273.32) (width 0.25) (layer "F.Cu") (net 1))
 (segment (start 202.254276 110.975) (end 193.479276 119.75) (width 0.25) (layer "F.Cu") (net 1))
 (segment (start 225.423808 267.785) (end 224.605 267.785) (width 0.25) (layer "F.Cu") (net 1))
 (segment (start 193.479276 119.75) (end 181.755 119.75) (width 0.25) (layer "F.Cu") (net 1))
 (segment (start 224.605 267.785) (end 224.155698 267.335698) (width 0.25) (layer "F.Cu") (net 1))
 (segment (start 148.629 119.75) (end 181.755 119.75) (width 16) (layer "F.Cu") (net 1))
 (segment (start 238.205 118.850276) (end 230.329724 110.975) (width 0.25) (layer "F.Cu") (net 1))
 (segment (start 227.59 272.338808) (end 227.59 269.951192) (width 0.25) (layer "F.Cu") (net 1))
 (segment (start 227.59 269.951192) (end 225.423808 267.785) (width 0.25) (layer "F.Cu") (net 1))
 (segment (start 230.329724 110.975) (end 202.254276 110.975) (width 0.25) (layer "F.Cu") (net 1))
 (segment (start 224.155 261.62) (end 238.205 247.57) (width 0.25) (layer "F.Cu") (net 1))
 (segment (start 224.155698 267.335698) (end 224.155698 261.620698) (width 0.25) (layer "F.Cu") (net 1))
 (segment (start 226.608808 273.32) (end 227.59 272.338808) (width 0.25) (layer "F.Cu") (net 1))
 (segment (start 224.155698 261.620698) (end 224.155 261.62) (width 0.25) (layer "F.Cu") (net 1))
 (segment (start 238.205 247.57) (end 238.205 118.850276) (width 0.25) (layer "F.Cu") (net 1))
 (segment (start 181.755 119.75) (end 148.629 119.75) (width 16) (layer "B.Cu") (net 1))
 (segment (start 204.915 271.145) (end 204.915 269.845) (width 0.25) (layer "F.Cu") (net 8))
 (segment (start 200.715 271.145) (end 204.915 271.145) (width 0.25) (layer "F.Cu") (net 8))
 (segment (start 200.715 265.645) (end 197.27 265.645) (width 0.25) (layer "F.Cu") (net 8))
 (segment (start 175.26 266.7) (end 182.88 266.7) (width 16) (layer "F.Cu") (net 8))
 (segment (start 200.715 265.645) (end 200.715 271.145) (width 0.25) (layer "F.Cu") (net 8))
 (segment (start 171.45 274.2175) (end 165.3335 280.334) (width 2.5) (layer "F.Cu") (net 8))
 (segment (start 204.915 269.845) (end 209.115 265.645) (width 0.25) (layer "F.Cu") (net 8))
 (segment (start 200.715 265.645) (end 209.115 265.645) (width 0.25) (layer "F.Cu") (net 8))
 (segment (start 165.3335 280.334) (end 135.554 280.334) (width 2.5) (layer "F.Cu") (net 8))
 (segment (start 197.27 265.645) (end 188.595 274.32) (width 0.25) (layer "F.Cu") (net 8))
 (segment (start 209.159 240.421) (end 226.695 240.421) (width 16) (layer "F.Cu") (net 8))
 (segment (start 182.88 266.7) (end 209.159 240.421) (width 16) (layer "F.Cu") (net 8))
 (segment (start 135.554 280.334) (end 132.715 277.495) (width 2.5) (layer "F.Cu") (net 8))
 (segment (start 182.88 266.7) (end 175.26 266.7) (width 16) (layer "B.Cu") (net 8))
 (segment (start 209.159 240.421) (end 182.88 266.7) (width 16) (layer "B.Cu") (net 8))
 (segment (start 226.695 240.421) (end 209.159 240.421) (width 16) (layer "B.Cu") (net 8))
 (segment (start 205.889 216.287) (end 181.755 240.421) (width 16) (layer "F.Cu") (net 10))
 (segment (start 226.695 216.287) (end 205.889 216.287) (width 16) (layer "F.Cu") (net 10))
 (segment (start 211.29 264.801192) (end 227.345192 248.746) (width 0.25) (layer "F.Cu") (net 10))
 (segment (start 235.02 243.869328) (end 235.02 224.612) (width 0.25) (layer "F.Cu") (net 10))
 (segment (start 235.02 224.612) (end 226.695 216.287) (width 0.25) (layer "F.Cu") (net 10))
 (segment (start 211.29 268.97) (end 211.29 264.801192) (width 0.25) (layer "F.Cu") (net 10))
 (segment (start 230.143328 248.746) (end 235.02 243.869328) (width 0.25) (layer "F.Cu") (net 10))
 (segment (start 209.115 271.145) (end 211.29 268.97) (width 0.25) (layer "F.Cu") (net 10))
 (segment (start 227.345192 248.746) (end 230.143328 248.746) (width 0.25) (layer "F.Cu") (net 10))
 (segment (start 226.695 216.287) (end 205.889 216.287) (width 16) (layer "B.Cu") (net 10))
 (segment (start 205.889 216.287) (end 181.755 240.421) (width 16) (layer "B.Cu") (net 10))
 (segment (start 236.855 182.245) (end 236.855 150.495) (width 0.25) (layer "F.Cu") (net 3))
 (segment (start 236.855 150.495) (end 236.855 149.225) (width 0.25) (layer "F.Cu") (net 3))
 (segment (start 236.855 149.86) (end 236.855 149.225) (width 0.25) (layer "F.Cu") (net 3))
 (segment (start 236.855 149.225) (end 236.855 129.91) (width 0.25) (layer "F.Cu") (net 3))
 (segment (start 236.855 129.91) (end 226.695 119.75) (width 0.25) (layer "F.Cu") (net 3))
 (segment (start 236.855 187.325) (end 236.855 149.86) (width 0.25) (layer "F.Cu") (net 3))
 (segment (start 236.855 247.015) (end 236.855 187.325) (width 0.25) (layer "F.Cu") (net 3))
 (segment (start 221.715 262.155) (end 236.855 247.015) (width 0.25) (layer "F.Cu") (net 3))
 (segment (start 236.82 182.245) (end 236.855 182.245) (width 0.25) (layer "F.Cu") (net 3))
 (segment (start 226.695 119.75) (end 205.889 119.75) (width 16) (layer "F.Cu") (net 3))
 (segment (start 236.855 187.325) (end 236.82 187.29) (width 0.25) (layer "F.Cu") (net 3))
 (segment (start 205.889 119.75) (end 181.755 143.884) (width 16) (layer "F.Cu") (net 3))
 (segment (start 236.82 187.29) (end 236.82 182.245) (width 0.25) (layer "F.Cu") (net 3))
 (segment (start 221.715 265.645) (end 221.715 262.155) (width 0.25) (layer "F.Cu") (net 3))
 (segment (start 236.855 150.495) (end 236.855 149.86) (width 0.25) (layer "F.Cu") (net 3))
 (segment (start 226.695 119.75) (end 205.889 119.75) (width 16) (layer "B.Cu") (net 3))
 (segment (start 205.889 119.75) (end 181.755 143.884) (width 16) (layer "B.Cu") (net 3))
 (segment (start 236.37 246.79) (end 236.37 153.559) (width 0.25) (layer "F.Cu") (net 6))
 (segment (start 226.695 143.884) (end 205.889 143.884) (width 16) (layer "F.Cu") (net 6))
 (segment (start 217.515 265.645) (end 236.37 246.79) (width 0.25) (layer "F.Cu") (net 6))
 (segment (start 236.37 153.559) (end 226.695 143.884) (width 0.25) (layer "F.Cu") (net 6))
 (segment (start 205.889 143.884) (end 181.755 168.018) (width 16) (layer "F.Cu") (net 6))
 (segment (start 217.515 271.145) (end 217.515 265.645) (width 0.25) (layer "F.Cu") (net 6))
 (segment (start 226.695 143.884) (end 205.889 143.884) (width 16) (layer "B.Cu") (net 6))
 (segment (start 205.889 143.884) (end 181.755 168.018) (width 16) (layer "B.Cu") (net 6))
 (segment (start 205.89 168.018) (end 181.755 192.153) (width 16) (layer "F.Cu") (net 5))
 (segment (start 215.49 268.97) (end 215.49 264.67212) (width 0.25) (layer "F.Cu") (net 5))
 (segment (start 235.92 177.243) (end 226.695 168.018) (width 0.25) (layer "F.Cu") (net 5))
 (segment (start 213.315 271.145) (end 215.49 268.97) (width 0.25) (layer "F.Cu") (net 5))
 (segment (start 235.92 244.24212) (end 235.92 177.243) (width 0.25) (layer "F.Cu") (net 5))
 (segment (start 215.49 264.67212) (end 235.92 244.24212) (width 0.25) (layer "F.Cu") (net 5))
 (segment (start 226.695 168.018) (end 205.89 168.018) (width 16) (layer "F.Cu") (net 5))
 (segment (start 226.695 168.018) (end 205.89 168.018) (width 16) (layer "B.Cu") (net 5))
 (segment (start 205.89 168.018) (end 181.755 192.153) (width 16) (layer "B.Cu") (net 5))
 (segment (start 205.889 192.153) (end 181.755 216.287) (width 16) (layer "F.Cu") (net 13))
 (segment (start 213.880724 265.645) (end 235.47 244.055724) (width 0.25) (layer "F.Cu") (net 13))
 (segment (start 235.47 200.928) (end 226.695 192.153) (width 0.25) (layer "F.Cu") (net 13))
 (segment (start 235.47 244.055724) (end 235.47 200.928) (width 0.25) (layer "F.Cu") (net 13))
 (segment (start 226.695 192.153) (end 205.889 192.153) (width 16) (layer "F.Cu") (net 13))
 (segment (start 213.315 265.645) (end 213.880724 265.645) (width 0.25) (layer "F.Cu") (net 13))
 (segment (start 205.889 192.153) (end 181.755 216.287) (width 16) (layer "B.Cu") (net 13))
 (segment (start 226.695 192.153) (end 205.889 192.153) (width 16) (layer "B.Cu") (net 13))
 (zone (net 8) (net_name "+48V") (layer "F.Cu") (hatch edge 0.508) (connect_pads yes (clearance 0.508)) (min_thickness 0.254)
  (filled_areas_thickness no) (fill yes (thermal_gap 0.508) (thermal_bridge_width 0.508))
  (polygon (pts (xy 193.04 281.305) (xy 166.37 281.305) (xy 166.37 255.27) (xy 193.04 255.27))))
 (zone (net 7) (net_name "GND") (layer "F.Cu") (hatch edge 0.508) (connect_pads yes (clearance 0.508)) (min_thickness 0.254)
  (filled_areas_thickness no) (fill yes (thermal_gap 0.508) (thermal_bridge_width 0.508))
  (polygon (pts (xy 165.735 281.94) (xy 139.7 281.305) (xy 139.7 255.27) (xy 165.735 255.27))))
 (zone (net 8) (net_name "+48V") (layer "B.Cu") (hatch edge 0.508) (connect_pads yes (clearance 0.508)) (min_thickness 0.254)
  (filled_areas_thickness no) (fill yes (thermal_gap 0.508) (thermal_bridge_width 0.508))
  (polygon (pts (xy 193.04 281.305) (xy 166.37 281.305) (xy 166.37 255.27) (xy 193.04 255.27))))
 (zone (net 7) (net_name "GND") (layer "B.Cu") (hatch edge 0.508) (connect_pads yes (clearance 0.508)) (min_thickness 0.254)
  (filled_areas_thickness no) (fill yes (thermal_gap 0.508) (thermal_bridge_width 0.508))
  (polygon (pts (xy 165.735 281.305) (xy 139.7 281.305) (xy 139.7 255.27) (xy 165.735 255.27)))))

